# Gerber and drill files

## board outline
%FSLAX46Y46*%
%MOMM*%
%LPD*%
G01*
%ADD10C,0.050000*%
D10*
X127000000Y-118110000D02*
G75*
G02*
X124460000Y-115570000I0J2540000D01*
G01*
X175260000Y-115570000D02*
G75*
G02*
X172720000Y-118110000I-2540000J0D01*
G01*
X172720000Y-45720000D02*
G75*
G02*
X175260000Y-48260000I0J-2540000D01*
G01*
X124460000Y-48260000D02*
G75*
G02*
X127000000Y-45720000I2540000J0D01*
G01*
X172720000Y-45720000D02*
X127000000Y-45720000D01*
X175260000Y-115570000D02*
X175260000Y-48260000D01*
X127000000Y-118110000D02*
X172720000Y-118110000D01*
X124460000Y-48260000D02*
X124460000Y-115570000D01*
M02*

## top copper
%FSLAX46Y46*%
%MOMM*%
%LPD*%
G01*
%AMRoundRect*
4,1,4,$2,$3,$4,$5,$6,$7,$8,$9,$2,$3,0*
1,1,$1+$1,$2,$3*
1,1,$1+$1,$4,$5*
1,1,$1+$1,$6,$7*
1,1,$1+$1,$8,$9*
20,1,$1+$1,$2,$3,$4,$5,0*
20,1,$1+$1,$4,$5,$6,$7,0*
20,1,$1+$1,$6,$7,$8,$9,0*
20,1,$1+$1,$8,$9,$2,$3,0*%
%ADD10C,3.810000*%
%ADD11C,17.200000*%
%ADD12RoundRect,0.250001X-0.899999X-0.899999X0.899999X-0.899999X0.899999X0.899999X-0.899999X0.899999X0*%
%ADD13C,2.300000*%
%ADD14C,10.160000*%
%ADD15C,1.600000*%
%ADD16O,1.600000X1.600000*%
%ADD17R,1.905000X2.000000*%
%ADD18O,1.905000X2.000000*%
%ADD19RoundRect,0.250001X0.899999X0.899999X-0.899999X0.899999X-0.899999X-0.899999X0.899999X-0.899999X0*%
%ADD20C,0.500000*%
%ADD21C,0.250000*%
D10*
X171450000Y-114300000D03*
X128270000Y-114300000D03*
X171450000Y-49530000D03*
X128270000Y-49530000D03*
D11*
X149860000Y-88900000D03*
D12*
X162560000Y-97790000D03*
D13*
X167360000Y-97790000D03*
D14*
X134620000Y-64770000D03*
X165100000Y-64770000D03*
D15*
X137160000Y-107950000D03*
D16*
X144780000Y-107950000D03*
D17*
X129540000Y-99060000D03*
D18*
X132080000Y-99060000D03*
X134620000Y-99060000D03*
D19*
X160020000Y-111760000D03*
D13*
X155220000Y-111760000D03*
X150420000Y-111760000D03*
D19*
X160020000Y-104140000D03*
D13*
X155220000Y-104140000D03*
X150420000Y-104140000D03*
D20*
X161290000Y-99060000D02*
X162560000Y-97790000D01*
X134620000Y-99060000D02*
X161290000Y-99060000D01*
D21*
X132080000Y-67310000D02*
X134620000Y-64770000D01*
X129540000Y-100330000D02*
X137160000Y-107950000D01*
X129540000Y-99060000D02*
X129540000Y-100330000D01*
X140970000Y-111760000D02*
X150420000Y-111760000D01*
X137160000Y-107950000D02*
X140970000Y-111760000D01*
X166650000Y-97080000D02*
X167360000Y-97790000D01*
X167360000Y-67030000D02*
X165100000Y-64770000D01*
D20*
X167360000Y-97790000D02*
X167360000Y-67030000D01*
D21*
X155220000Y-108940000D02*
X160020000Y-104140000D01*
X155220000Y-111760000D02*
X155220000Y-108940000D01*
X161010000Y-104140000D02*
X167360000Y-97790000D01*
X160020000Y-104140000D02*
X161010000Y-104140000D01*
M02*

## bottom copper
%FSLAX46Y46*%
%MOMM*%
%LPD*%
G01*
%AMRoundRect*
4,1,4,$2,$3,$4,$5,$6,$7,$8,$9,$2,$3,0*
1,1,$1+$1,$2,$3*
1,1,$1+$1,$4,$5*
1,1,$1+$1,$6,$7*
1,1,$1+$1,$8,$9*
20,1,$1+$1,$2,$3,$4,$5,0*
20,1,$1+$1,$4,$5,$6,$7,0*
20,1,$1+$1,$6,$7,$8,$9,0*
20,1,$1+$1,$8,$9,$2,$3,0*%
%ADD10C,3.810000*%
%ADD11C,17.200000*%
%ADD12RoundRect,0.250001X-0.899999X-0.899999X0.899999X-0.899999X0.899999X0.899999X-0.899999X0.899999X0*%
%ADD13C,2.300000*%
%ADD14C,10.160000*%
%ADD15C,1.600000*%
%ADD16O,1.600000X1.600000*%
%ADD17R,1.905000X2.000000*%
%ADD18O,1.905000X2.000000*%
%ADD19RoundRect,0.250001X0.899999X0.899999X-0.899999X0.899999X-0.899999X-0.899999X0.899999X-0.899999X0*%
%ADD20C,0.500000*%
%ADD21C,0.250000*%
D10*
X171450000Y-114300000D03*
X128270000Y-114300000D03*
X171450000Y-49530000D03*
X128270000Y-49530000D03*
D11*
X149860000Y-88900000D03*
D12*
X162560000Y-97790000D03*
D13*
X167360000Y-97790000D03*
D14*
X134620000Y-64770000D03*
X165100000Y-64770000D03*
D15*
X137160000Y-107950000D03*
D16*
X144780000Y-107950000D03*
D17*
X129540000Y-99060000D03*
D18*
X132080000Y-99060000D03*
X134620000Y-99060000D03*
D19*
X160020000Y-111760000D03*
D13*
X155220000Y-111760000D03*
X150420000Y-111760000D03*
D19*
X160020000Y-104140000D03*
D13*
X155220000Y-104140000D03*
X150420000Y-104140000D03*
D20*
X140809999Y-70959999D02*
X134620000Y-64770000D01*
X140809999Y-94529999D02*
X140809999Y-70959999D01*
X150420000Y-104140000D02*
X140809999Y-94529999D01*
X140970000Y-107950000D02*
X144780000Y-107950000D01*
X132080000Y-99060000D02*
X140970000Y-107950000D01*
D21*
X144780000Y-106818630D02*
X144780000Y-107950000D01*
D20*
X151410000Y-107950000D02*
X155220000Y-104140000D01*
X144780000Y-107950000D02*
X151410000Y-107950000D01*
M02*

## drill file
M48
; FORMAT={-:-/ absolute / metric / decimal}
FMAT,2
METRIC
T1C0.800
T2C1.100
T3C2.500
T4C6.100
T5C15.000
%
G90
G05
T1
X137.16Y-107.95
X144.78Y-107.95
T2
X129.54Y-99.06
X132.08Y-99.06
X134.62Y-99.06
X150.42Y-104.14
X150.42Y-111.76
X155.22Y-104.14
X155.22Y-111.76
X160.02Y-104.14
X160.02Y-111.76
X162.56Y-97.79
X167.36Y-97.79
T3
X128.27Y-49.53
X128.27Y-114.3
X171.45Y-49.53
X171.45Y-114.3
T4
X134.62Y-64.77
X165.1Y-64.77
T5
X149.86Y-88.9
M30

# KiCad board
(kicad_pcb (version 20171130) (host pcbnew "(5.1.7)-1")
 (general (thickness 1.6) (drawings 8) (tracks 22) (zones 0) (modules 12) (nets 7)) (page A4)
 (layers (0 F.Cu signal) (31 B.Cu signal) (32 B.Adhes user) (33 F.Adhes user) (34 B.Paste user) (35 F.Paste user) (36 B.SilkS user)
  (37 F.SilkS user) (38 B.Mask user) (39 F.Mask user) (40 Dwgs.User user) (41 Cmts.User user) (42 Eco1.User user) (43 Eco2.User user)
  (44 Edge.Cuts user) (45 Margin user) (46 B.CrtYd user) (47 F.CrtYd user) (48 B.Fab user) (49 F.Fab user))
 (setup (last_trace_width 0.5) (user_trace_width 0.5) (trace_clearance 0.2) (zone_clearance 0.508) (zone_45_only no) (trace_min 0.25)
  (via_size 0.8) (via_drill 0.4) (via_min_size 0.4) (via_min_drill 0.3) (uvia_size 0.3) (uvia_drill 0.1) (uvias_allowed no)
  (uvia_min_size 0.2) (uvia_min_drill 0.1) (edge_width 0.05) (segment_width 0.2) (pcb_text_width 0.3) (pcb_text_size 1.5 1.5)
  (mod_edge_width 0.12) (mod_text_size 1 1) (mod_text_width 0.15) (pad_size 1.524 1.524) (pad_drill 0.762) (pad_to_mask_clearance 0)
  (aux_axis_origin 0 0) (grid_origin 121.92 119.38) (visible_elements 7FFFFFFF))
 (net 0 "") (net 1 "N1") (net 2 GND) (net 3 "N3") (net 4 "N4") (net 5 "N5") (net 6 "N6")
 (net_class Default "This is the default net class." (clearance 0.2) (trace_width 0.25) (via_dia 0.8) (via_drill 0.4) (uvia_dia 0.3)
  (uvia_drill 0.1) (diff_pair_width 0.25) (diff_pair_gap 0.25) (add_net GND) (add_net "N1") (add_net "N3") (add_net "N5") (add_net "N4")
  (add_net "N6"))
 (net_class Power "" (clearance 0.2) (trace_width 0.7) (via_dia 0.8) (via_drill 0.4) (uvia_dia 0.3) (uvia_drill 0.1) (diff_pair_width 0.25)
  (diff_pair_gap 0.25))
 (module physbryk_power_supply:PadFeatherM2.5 (layer F.Cu) (at 171.45 114.3)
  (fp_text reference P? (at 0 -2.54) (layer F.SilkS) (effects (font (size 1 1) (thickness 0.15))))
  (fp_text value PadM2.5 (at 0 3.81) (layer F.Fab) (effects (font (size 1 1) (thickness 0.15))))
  (pad ? thru_hole circle (at 0 0) (size 3.81 3.81) (drill 2.5) (layers *.Cu *.Mask) (solder_mask_margin 0.0508)))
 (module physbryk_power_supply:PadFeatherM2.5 (layer F.Cu) (at 128.27 114.3)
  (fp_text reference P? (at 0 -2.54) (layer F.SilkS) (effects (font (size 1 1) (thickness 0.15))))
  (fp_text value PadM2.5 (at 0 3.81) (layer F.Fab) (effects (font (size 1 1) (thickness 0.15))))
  (pad ? thru_hole circle (at 0 0) (size 3.81 3.81) (drill 2.5) (layers *.Cu *.Mask) (solder_mask_margin 0.0508)))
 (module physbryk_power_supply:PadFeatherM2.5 (layer F.Cu) (at 171.45 49.53)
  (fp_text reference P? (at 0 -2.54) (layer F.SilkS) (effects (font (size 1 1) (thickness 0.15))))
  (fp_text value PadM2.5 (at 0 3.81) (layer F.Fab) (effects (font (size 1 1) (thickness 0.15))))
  (pad ? thru_hole circle (at 0 0) (size 3.81 3.81) (drill 2.5) (layers *.Cu *.Mask) (solder_mask_margin 0.0508)))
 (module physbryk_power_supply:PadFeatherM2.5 (layer F.Cu) (at 128.27 49.53)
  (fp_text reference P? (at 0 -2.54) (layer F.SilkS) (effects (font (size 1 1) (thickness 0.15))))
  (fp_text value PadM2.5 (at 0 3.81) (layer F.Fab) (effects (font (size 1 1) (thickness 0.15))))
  (pad ? thru_hole circle (at 0 0) (size 3.81 3.81) (drill 2.5) (layers *.Cu *.Mask) (solder_mask_margin 0.0508)))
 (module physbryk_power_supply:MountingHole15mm (layer F.Cu) (at 149.86 88.9)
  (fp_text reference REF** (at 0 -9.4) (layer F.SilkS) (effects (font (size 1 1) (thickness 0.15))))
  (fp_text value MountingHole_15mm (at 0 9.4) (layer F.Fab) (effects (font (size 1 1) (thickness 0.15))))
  (pad 1 thru_hole circle (at 0 0) (size 17.2 17.2) (drill 15) (layers *.Cu *.Mask)))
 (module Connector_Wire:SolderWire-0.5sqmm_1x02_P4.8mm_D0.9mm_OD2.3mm (layer F.Cu) (at 162.56 97.79)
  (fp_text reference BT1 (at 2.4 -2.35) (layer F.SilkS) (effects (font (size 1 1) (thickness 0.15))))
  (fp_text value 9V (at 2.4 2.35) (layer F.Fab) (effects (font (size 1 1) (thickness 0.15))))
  (pad 1 thru_hole roundrect (at 0 0) (size 2.3 2.3) (drill 1.1) (layers *.Cu *.Mask) (roundrect_rratio 0.108696) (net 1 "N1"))
  (pad 2 thru_hole circle (at 4.8 0) (size 2.3 2.3) (drill 1.1) (layers *.Cu *.Mask) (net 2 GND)))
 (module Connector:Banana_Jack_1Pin (layer F.Cu) (at 134.62 64.77)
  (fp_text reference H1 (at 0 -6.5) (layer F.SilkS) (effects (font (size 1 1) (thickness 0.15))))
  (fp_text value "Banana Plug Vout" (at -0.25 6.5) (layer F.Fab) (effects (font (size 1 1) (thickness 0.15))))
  (pad 1 thru_hole circle (at 0 0) (size 10.16 10.16) (drill 6.1) (layers *.Cu *.Mask) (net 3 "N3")))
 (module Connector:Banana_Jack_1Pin (layer F.Cu) (at 165.1 64.77)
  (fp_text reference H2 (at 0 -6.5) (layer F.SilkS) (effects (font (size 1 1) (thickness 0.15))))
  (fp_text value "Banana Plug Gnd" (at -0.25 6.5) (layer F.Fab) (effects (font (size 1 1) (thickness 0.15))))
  (pad 1 thru_hole circle (at 0 0) (size 10.16 10.16) (drill 6.1) (layers *.Cu *.Mask) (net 2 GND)))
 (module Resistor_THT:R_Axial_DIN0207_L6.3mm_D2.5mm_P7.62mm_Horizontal (layer F.Cu) (at 137.16 107.95)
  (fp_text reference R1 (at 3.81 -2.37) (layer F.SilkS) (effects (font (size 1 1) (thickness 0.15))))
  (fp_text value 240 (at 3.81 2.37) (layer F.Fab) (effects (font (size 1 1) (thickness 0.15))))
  (pad 1 thru_hole circle (at 0 0) (size 1.6 1.6) (drill 0.8) (layers *.Cu *.Mask) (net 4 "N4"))
  (pad 2 thru_hole oval (at 7.62 0) (size 1.6 1.6) (drill 0.8) (layers *.Cu *.Mask) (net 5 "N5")))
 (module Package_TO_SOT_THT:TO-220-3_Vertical (layer F.Cu) (at 129.54 99.06)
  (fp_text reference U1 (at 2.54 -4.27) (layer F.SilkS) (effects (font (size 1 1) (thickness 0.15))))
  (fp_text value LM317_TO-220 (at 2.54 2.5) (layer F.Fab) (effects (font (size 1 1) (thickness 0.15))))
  (pad 1 thru_hole rect (at 0 0) (size 1.905 2) (drill 1.1) (layers *.Cu *.Mask) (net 4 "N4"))
  (pad 2 thru_hole oval (at 2.54 0) (size 1.905 2) (drill 1.1) (layers *.Cu *.Mask) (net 5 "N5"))
  (pad 3 thru_hole oval (at 5.08 0) (size 1.905 2) (drill 1.1) (layers *.Cu *.Mask) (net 1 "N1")))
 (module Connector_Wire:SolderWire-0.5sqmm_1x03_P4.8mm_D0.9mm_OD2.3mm (layer F.Cu) (at 160.02 111.76 180)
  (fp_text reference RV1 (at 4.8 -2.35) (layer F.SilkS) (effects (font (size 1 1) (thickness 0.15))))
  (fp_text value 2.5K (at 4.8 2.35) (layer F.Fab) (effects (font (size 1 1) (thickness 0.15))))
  (pad 1 thru_hole roundrect (at 0 0 180) (size 2.3 2.3) (drill 1.1) (layers *.Cu *.Mask) (roundrect_rratio 0.108696) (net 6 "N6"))
  (pad 2 thru_hole circle (at 4.8 0 180) (size 2.3 2.3) (drill 1.1) (layers *.Cu *.Mask) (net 2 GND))
  (pad 3 thru_hole circle (at 9.6 0 180) (size 2.3 2.3) (drill 1.1) (layers *.Cu *.Mask) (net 4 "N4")))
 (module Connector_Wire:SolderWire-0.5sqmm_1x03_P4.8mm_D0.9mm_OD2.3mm (layer F.Cu) (at 160.02 104.14 180)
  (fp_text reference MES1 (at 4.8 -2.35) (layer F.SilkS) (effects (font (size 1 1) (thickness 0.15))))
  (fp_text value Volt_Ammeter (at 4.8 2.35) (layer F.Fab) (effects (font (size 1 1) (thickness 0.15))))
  (pad 1 thru_hole roundrect (at 0 0 180) (size 2.3 2.3) (drill 1.1) (layers *.Cu *.Mask) (roundrect_rratio 0.108696) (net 2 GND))
  (pad 2 thru_hole circle (at 4.8 0 180) (size 2.3 2.3) (drill 1.1) (layers *.Cu *.Mask) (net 5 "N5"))
  (pad 3 thru_hole circle (at 9.6 0 180) (size 2.3 2.3) (drill 1.1) (layers *.Cu *.Mask) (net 3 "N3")))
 (gr_arc (start 127 115.57) (end 124.46 115.57) (angle -90) (layer Edge.Cuts) (width 0.05))
 (gr_arc (start 172.72 115.57) (end 172.72 118.11) (angle -90) (layer Edge.Cuts) (width 0.05))
 (gr_arc (start 172.72 48.26) (end 175.26 48.26) (angle -90) (layer Edge.Cuts) (width 0.05))
 (gr_arc (start 127 48.26) (end 127 45.72) (angle -90) (layer Edge.Cuts) (width 0.05))
 (gr_line (start 172.72 45.72) (end 127 45.72) (layer Edge.Cuts) (width 0.05))
 (gr_line (start 175.26 115.57) (end 175.26 48.26) (layer Edge.Cuts) (width 0.05))
 (gr_line (start 127 118.11) (end 172.72 118.11) (layer Edge.Cuts) (width 0.05))
 (gr_line (start 124.46 48.26) (end 124.46 115.57) (layer Edge.Cuts) (width 0.05))
 (segment (start 161.29 99.06) (end 162.56 97.79) (width 0.5) (layer F.Cu) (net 1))
 (segment (start 134.62 99.06) (end 161.29 99.06) (width 0.5) (layer F.Cu) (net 1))
 (segment (start 132.08 67.31) (end 134.62 64.77) (width 0.25) (layer F.Cu) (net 3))
 (segment (start 140.809999 70.959999) (end 134.62 64.77) (width 0.5) (layer B.Cu) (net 3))
 (segment (start 140.809999 94.529999) (end 140.809999 70.959999) (width 0.5) (layer B.Cu) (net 3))
 (segment (start 150.42 104.14) (end 140.809999 94.529999) (width 0.5) (layer B.Cu) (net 3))
 (segment (start 129.54 100.33) (end 137.16 107.95) (width 0.25) (layer F.Cu) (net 4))
 (segment (start 129.54 99.06) (end 129.54 100.33) (width 0.25) (layer F.Cu) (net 4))
 (segment (start 140.97 111.76) (end 150.42 111.76) (width 0.25) (layer F.Cu) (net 4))
 (segment (start 137.16 107.95) (end 140.97 111.76) (width 0.25) (layer F.Cu) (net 4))
 (segment (start 166.65 97.08) (end 167.36 97.79) (width 0.25) (layer F.Cu) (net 2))
 (segment (start 167.36 67.03) (end 165.1 64.77) (width 0.25) (layer F.Cu) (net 2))
 (segment (start 167.36 97.79) (end 167.36 67.03) (width 0.5) (layer F.Cu) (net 2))
 (segment (start 155.22 108.94) (end 160.02 104.14) (width 0.25) (layer F.Cu) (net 2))
 (segment (start 155.22 111.76) (end 155.22 108.94) (width 0.25) (layer F.Cu) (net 2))
 (segment (start 161.01 104.14) (end 167.36 97.79) (width 0.25) (layer F.Cu) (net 2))
 (segment (start 160.02 104.14) (end 161.01 104.14) (width 0.25) (layer F.Cu) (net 2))
 (segment (start 140.97 107.95) (end 144.78 107.95) (width 0.5) (layer B.Cu) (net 5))
 (segment (start 132.08 99.06) (end 140.97 107.95) (width 0.5) (layer B.Cu) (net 5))
 (segment (start 144.78 106.81863) (end 144.78 107.95) (width 0.25) (layer B.Cu) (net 5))
 (segment (start 151.41 107.95) (end 155.22 104.14) (width 0.5) (layer B.Cu) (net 5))
 (segment (start 144.78 107.95) (end 151.41 107.95) (width 0.5) (layer B.Cu) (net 5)))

